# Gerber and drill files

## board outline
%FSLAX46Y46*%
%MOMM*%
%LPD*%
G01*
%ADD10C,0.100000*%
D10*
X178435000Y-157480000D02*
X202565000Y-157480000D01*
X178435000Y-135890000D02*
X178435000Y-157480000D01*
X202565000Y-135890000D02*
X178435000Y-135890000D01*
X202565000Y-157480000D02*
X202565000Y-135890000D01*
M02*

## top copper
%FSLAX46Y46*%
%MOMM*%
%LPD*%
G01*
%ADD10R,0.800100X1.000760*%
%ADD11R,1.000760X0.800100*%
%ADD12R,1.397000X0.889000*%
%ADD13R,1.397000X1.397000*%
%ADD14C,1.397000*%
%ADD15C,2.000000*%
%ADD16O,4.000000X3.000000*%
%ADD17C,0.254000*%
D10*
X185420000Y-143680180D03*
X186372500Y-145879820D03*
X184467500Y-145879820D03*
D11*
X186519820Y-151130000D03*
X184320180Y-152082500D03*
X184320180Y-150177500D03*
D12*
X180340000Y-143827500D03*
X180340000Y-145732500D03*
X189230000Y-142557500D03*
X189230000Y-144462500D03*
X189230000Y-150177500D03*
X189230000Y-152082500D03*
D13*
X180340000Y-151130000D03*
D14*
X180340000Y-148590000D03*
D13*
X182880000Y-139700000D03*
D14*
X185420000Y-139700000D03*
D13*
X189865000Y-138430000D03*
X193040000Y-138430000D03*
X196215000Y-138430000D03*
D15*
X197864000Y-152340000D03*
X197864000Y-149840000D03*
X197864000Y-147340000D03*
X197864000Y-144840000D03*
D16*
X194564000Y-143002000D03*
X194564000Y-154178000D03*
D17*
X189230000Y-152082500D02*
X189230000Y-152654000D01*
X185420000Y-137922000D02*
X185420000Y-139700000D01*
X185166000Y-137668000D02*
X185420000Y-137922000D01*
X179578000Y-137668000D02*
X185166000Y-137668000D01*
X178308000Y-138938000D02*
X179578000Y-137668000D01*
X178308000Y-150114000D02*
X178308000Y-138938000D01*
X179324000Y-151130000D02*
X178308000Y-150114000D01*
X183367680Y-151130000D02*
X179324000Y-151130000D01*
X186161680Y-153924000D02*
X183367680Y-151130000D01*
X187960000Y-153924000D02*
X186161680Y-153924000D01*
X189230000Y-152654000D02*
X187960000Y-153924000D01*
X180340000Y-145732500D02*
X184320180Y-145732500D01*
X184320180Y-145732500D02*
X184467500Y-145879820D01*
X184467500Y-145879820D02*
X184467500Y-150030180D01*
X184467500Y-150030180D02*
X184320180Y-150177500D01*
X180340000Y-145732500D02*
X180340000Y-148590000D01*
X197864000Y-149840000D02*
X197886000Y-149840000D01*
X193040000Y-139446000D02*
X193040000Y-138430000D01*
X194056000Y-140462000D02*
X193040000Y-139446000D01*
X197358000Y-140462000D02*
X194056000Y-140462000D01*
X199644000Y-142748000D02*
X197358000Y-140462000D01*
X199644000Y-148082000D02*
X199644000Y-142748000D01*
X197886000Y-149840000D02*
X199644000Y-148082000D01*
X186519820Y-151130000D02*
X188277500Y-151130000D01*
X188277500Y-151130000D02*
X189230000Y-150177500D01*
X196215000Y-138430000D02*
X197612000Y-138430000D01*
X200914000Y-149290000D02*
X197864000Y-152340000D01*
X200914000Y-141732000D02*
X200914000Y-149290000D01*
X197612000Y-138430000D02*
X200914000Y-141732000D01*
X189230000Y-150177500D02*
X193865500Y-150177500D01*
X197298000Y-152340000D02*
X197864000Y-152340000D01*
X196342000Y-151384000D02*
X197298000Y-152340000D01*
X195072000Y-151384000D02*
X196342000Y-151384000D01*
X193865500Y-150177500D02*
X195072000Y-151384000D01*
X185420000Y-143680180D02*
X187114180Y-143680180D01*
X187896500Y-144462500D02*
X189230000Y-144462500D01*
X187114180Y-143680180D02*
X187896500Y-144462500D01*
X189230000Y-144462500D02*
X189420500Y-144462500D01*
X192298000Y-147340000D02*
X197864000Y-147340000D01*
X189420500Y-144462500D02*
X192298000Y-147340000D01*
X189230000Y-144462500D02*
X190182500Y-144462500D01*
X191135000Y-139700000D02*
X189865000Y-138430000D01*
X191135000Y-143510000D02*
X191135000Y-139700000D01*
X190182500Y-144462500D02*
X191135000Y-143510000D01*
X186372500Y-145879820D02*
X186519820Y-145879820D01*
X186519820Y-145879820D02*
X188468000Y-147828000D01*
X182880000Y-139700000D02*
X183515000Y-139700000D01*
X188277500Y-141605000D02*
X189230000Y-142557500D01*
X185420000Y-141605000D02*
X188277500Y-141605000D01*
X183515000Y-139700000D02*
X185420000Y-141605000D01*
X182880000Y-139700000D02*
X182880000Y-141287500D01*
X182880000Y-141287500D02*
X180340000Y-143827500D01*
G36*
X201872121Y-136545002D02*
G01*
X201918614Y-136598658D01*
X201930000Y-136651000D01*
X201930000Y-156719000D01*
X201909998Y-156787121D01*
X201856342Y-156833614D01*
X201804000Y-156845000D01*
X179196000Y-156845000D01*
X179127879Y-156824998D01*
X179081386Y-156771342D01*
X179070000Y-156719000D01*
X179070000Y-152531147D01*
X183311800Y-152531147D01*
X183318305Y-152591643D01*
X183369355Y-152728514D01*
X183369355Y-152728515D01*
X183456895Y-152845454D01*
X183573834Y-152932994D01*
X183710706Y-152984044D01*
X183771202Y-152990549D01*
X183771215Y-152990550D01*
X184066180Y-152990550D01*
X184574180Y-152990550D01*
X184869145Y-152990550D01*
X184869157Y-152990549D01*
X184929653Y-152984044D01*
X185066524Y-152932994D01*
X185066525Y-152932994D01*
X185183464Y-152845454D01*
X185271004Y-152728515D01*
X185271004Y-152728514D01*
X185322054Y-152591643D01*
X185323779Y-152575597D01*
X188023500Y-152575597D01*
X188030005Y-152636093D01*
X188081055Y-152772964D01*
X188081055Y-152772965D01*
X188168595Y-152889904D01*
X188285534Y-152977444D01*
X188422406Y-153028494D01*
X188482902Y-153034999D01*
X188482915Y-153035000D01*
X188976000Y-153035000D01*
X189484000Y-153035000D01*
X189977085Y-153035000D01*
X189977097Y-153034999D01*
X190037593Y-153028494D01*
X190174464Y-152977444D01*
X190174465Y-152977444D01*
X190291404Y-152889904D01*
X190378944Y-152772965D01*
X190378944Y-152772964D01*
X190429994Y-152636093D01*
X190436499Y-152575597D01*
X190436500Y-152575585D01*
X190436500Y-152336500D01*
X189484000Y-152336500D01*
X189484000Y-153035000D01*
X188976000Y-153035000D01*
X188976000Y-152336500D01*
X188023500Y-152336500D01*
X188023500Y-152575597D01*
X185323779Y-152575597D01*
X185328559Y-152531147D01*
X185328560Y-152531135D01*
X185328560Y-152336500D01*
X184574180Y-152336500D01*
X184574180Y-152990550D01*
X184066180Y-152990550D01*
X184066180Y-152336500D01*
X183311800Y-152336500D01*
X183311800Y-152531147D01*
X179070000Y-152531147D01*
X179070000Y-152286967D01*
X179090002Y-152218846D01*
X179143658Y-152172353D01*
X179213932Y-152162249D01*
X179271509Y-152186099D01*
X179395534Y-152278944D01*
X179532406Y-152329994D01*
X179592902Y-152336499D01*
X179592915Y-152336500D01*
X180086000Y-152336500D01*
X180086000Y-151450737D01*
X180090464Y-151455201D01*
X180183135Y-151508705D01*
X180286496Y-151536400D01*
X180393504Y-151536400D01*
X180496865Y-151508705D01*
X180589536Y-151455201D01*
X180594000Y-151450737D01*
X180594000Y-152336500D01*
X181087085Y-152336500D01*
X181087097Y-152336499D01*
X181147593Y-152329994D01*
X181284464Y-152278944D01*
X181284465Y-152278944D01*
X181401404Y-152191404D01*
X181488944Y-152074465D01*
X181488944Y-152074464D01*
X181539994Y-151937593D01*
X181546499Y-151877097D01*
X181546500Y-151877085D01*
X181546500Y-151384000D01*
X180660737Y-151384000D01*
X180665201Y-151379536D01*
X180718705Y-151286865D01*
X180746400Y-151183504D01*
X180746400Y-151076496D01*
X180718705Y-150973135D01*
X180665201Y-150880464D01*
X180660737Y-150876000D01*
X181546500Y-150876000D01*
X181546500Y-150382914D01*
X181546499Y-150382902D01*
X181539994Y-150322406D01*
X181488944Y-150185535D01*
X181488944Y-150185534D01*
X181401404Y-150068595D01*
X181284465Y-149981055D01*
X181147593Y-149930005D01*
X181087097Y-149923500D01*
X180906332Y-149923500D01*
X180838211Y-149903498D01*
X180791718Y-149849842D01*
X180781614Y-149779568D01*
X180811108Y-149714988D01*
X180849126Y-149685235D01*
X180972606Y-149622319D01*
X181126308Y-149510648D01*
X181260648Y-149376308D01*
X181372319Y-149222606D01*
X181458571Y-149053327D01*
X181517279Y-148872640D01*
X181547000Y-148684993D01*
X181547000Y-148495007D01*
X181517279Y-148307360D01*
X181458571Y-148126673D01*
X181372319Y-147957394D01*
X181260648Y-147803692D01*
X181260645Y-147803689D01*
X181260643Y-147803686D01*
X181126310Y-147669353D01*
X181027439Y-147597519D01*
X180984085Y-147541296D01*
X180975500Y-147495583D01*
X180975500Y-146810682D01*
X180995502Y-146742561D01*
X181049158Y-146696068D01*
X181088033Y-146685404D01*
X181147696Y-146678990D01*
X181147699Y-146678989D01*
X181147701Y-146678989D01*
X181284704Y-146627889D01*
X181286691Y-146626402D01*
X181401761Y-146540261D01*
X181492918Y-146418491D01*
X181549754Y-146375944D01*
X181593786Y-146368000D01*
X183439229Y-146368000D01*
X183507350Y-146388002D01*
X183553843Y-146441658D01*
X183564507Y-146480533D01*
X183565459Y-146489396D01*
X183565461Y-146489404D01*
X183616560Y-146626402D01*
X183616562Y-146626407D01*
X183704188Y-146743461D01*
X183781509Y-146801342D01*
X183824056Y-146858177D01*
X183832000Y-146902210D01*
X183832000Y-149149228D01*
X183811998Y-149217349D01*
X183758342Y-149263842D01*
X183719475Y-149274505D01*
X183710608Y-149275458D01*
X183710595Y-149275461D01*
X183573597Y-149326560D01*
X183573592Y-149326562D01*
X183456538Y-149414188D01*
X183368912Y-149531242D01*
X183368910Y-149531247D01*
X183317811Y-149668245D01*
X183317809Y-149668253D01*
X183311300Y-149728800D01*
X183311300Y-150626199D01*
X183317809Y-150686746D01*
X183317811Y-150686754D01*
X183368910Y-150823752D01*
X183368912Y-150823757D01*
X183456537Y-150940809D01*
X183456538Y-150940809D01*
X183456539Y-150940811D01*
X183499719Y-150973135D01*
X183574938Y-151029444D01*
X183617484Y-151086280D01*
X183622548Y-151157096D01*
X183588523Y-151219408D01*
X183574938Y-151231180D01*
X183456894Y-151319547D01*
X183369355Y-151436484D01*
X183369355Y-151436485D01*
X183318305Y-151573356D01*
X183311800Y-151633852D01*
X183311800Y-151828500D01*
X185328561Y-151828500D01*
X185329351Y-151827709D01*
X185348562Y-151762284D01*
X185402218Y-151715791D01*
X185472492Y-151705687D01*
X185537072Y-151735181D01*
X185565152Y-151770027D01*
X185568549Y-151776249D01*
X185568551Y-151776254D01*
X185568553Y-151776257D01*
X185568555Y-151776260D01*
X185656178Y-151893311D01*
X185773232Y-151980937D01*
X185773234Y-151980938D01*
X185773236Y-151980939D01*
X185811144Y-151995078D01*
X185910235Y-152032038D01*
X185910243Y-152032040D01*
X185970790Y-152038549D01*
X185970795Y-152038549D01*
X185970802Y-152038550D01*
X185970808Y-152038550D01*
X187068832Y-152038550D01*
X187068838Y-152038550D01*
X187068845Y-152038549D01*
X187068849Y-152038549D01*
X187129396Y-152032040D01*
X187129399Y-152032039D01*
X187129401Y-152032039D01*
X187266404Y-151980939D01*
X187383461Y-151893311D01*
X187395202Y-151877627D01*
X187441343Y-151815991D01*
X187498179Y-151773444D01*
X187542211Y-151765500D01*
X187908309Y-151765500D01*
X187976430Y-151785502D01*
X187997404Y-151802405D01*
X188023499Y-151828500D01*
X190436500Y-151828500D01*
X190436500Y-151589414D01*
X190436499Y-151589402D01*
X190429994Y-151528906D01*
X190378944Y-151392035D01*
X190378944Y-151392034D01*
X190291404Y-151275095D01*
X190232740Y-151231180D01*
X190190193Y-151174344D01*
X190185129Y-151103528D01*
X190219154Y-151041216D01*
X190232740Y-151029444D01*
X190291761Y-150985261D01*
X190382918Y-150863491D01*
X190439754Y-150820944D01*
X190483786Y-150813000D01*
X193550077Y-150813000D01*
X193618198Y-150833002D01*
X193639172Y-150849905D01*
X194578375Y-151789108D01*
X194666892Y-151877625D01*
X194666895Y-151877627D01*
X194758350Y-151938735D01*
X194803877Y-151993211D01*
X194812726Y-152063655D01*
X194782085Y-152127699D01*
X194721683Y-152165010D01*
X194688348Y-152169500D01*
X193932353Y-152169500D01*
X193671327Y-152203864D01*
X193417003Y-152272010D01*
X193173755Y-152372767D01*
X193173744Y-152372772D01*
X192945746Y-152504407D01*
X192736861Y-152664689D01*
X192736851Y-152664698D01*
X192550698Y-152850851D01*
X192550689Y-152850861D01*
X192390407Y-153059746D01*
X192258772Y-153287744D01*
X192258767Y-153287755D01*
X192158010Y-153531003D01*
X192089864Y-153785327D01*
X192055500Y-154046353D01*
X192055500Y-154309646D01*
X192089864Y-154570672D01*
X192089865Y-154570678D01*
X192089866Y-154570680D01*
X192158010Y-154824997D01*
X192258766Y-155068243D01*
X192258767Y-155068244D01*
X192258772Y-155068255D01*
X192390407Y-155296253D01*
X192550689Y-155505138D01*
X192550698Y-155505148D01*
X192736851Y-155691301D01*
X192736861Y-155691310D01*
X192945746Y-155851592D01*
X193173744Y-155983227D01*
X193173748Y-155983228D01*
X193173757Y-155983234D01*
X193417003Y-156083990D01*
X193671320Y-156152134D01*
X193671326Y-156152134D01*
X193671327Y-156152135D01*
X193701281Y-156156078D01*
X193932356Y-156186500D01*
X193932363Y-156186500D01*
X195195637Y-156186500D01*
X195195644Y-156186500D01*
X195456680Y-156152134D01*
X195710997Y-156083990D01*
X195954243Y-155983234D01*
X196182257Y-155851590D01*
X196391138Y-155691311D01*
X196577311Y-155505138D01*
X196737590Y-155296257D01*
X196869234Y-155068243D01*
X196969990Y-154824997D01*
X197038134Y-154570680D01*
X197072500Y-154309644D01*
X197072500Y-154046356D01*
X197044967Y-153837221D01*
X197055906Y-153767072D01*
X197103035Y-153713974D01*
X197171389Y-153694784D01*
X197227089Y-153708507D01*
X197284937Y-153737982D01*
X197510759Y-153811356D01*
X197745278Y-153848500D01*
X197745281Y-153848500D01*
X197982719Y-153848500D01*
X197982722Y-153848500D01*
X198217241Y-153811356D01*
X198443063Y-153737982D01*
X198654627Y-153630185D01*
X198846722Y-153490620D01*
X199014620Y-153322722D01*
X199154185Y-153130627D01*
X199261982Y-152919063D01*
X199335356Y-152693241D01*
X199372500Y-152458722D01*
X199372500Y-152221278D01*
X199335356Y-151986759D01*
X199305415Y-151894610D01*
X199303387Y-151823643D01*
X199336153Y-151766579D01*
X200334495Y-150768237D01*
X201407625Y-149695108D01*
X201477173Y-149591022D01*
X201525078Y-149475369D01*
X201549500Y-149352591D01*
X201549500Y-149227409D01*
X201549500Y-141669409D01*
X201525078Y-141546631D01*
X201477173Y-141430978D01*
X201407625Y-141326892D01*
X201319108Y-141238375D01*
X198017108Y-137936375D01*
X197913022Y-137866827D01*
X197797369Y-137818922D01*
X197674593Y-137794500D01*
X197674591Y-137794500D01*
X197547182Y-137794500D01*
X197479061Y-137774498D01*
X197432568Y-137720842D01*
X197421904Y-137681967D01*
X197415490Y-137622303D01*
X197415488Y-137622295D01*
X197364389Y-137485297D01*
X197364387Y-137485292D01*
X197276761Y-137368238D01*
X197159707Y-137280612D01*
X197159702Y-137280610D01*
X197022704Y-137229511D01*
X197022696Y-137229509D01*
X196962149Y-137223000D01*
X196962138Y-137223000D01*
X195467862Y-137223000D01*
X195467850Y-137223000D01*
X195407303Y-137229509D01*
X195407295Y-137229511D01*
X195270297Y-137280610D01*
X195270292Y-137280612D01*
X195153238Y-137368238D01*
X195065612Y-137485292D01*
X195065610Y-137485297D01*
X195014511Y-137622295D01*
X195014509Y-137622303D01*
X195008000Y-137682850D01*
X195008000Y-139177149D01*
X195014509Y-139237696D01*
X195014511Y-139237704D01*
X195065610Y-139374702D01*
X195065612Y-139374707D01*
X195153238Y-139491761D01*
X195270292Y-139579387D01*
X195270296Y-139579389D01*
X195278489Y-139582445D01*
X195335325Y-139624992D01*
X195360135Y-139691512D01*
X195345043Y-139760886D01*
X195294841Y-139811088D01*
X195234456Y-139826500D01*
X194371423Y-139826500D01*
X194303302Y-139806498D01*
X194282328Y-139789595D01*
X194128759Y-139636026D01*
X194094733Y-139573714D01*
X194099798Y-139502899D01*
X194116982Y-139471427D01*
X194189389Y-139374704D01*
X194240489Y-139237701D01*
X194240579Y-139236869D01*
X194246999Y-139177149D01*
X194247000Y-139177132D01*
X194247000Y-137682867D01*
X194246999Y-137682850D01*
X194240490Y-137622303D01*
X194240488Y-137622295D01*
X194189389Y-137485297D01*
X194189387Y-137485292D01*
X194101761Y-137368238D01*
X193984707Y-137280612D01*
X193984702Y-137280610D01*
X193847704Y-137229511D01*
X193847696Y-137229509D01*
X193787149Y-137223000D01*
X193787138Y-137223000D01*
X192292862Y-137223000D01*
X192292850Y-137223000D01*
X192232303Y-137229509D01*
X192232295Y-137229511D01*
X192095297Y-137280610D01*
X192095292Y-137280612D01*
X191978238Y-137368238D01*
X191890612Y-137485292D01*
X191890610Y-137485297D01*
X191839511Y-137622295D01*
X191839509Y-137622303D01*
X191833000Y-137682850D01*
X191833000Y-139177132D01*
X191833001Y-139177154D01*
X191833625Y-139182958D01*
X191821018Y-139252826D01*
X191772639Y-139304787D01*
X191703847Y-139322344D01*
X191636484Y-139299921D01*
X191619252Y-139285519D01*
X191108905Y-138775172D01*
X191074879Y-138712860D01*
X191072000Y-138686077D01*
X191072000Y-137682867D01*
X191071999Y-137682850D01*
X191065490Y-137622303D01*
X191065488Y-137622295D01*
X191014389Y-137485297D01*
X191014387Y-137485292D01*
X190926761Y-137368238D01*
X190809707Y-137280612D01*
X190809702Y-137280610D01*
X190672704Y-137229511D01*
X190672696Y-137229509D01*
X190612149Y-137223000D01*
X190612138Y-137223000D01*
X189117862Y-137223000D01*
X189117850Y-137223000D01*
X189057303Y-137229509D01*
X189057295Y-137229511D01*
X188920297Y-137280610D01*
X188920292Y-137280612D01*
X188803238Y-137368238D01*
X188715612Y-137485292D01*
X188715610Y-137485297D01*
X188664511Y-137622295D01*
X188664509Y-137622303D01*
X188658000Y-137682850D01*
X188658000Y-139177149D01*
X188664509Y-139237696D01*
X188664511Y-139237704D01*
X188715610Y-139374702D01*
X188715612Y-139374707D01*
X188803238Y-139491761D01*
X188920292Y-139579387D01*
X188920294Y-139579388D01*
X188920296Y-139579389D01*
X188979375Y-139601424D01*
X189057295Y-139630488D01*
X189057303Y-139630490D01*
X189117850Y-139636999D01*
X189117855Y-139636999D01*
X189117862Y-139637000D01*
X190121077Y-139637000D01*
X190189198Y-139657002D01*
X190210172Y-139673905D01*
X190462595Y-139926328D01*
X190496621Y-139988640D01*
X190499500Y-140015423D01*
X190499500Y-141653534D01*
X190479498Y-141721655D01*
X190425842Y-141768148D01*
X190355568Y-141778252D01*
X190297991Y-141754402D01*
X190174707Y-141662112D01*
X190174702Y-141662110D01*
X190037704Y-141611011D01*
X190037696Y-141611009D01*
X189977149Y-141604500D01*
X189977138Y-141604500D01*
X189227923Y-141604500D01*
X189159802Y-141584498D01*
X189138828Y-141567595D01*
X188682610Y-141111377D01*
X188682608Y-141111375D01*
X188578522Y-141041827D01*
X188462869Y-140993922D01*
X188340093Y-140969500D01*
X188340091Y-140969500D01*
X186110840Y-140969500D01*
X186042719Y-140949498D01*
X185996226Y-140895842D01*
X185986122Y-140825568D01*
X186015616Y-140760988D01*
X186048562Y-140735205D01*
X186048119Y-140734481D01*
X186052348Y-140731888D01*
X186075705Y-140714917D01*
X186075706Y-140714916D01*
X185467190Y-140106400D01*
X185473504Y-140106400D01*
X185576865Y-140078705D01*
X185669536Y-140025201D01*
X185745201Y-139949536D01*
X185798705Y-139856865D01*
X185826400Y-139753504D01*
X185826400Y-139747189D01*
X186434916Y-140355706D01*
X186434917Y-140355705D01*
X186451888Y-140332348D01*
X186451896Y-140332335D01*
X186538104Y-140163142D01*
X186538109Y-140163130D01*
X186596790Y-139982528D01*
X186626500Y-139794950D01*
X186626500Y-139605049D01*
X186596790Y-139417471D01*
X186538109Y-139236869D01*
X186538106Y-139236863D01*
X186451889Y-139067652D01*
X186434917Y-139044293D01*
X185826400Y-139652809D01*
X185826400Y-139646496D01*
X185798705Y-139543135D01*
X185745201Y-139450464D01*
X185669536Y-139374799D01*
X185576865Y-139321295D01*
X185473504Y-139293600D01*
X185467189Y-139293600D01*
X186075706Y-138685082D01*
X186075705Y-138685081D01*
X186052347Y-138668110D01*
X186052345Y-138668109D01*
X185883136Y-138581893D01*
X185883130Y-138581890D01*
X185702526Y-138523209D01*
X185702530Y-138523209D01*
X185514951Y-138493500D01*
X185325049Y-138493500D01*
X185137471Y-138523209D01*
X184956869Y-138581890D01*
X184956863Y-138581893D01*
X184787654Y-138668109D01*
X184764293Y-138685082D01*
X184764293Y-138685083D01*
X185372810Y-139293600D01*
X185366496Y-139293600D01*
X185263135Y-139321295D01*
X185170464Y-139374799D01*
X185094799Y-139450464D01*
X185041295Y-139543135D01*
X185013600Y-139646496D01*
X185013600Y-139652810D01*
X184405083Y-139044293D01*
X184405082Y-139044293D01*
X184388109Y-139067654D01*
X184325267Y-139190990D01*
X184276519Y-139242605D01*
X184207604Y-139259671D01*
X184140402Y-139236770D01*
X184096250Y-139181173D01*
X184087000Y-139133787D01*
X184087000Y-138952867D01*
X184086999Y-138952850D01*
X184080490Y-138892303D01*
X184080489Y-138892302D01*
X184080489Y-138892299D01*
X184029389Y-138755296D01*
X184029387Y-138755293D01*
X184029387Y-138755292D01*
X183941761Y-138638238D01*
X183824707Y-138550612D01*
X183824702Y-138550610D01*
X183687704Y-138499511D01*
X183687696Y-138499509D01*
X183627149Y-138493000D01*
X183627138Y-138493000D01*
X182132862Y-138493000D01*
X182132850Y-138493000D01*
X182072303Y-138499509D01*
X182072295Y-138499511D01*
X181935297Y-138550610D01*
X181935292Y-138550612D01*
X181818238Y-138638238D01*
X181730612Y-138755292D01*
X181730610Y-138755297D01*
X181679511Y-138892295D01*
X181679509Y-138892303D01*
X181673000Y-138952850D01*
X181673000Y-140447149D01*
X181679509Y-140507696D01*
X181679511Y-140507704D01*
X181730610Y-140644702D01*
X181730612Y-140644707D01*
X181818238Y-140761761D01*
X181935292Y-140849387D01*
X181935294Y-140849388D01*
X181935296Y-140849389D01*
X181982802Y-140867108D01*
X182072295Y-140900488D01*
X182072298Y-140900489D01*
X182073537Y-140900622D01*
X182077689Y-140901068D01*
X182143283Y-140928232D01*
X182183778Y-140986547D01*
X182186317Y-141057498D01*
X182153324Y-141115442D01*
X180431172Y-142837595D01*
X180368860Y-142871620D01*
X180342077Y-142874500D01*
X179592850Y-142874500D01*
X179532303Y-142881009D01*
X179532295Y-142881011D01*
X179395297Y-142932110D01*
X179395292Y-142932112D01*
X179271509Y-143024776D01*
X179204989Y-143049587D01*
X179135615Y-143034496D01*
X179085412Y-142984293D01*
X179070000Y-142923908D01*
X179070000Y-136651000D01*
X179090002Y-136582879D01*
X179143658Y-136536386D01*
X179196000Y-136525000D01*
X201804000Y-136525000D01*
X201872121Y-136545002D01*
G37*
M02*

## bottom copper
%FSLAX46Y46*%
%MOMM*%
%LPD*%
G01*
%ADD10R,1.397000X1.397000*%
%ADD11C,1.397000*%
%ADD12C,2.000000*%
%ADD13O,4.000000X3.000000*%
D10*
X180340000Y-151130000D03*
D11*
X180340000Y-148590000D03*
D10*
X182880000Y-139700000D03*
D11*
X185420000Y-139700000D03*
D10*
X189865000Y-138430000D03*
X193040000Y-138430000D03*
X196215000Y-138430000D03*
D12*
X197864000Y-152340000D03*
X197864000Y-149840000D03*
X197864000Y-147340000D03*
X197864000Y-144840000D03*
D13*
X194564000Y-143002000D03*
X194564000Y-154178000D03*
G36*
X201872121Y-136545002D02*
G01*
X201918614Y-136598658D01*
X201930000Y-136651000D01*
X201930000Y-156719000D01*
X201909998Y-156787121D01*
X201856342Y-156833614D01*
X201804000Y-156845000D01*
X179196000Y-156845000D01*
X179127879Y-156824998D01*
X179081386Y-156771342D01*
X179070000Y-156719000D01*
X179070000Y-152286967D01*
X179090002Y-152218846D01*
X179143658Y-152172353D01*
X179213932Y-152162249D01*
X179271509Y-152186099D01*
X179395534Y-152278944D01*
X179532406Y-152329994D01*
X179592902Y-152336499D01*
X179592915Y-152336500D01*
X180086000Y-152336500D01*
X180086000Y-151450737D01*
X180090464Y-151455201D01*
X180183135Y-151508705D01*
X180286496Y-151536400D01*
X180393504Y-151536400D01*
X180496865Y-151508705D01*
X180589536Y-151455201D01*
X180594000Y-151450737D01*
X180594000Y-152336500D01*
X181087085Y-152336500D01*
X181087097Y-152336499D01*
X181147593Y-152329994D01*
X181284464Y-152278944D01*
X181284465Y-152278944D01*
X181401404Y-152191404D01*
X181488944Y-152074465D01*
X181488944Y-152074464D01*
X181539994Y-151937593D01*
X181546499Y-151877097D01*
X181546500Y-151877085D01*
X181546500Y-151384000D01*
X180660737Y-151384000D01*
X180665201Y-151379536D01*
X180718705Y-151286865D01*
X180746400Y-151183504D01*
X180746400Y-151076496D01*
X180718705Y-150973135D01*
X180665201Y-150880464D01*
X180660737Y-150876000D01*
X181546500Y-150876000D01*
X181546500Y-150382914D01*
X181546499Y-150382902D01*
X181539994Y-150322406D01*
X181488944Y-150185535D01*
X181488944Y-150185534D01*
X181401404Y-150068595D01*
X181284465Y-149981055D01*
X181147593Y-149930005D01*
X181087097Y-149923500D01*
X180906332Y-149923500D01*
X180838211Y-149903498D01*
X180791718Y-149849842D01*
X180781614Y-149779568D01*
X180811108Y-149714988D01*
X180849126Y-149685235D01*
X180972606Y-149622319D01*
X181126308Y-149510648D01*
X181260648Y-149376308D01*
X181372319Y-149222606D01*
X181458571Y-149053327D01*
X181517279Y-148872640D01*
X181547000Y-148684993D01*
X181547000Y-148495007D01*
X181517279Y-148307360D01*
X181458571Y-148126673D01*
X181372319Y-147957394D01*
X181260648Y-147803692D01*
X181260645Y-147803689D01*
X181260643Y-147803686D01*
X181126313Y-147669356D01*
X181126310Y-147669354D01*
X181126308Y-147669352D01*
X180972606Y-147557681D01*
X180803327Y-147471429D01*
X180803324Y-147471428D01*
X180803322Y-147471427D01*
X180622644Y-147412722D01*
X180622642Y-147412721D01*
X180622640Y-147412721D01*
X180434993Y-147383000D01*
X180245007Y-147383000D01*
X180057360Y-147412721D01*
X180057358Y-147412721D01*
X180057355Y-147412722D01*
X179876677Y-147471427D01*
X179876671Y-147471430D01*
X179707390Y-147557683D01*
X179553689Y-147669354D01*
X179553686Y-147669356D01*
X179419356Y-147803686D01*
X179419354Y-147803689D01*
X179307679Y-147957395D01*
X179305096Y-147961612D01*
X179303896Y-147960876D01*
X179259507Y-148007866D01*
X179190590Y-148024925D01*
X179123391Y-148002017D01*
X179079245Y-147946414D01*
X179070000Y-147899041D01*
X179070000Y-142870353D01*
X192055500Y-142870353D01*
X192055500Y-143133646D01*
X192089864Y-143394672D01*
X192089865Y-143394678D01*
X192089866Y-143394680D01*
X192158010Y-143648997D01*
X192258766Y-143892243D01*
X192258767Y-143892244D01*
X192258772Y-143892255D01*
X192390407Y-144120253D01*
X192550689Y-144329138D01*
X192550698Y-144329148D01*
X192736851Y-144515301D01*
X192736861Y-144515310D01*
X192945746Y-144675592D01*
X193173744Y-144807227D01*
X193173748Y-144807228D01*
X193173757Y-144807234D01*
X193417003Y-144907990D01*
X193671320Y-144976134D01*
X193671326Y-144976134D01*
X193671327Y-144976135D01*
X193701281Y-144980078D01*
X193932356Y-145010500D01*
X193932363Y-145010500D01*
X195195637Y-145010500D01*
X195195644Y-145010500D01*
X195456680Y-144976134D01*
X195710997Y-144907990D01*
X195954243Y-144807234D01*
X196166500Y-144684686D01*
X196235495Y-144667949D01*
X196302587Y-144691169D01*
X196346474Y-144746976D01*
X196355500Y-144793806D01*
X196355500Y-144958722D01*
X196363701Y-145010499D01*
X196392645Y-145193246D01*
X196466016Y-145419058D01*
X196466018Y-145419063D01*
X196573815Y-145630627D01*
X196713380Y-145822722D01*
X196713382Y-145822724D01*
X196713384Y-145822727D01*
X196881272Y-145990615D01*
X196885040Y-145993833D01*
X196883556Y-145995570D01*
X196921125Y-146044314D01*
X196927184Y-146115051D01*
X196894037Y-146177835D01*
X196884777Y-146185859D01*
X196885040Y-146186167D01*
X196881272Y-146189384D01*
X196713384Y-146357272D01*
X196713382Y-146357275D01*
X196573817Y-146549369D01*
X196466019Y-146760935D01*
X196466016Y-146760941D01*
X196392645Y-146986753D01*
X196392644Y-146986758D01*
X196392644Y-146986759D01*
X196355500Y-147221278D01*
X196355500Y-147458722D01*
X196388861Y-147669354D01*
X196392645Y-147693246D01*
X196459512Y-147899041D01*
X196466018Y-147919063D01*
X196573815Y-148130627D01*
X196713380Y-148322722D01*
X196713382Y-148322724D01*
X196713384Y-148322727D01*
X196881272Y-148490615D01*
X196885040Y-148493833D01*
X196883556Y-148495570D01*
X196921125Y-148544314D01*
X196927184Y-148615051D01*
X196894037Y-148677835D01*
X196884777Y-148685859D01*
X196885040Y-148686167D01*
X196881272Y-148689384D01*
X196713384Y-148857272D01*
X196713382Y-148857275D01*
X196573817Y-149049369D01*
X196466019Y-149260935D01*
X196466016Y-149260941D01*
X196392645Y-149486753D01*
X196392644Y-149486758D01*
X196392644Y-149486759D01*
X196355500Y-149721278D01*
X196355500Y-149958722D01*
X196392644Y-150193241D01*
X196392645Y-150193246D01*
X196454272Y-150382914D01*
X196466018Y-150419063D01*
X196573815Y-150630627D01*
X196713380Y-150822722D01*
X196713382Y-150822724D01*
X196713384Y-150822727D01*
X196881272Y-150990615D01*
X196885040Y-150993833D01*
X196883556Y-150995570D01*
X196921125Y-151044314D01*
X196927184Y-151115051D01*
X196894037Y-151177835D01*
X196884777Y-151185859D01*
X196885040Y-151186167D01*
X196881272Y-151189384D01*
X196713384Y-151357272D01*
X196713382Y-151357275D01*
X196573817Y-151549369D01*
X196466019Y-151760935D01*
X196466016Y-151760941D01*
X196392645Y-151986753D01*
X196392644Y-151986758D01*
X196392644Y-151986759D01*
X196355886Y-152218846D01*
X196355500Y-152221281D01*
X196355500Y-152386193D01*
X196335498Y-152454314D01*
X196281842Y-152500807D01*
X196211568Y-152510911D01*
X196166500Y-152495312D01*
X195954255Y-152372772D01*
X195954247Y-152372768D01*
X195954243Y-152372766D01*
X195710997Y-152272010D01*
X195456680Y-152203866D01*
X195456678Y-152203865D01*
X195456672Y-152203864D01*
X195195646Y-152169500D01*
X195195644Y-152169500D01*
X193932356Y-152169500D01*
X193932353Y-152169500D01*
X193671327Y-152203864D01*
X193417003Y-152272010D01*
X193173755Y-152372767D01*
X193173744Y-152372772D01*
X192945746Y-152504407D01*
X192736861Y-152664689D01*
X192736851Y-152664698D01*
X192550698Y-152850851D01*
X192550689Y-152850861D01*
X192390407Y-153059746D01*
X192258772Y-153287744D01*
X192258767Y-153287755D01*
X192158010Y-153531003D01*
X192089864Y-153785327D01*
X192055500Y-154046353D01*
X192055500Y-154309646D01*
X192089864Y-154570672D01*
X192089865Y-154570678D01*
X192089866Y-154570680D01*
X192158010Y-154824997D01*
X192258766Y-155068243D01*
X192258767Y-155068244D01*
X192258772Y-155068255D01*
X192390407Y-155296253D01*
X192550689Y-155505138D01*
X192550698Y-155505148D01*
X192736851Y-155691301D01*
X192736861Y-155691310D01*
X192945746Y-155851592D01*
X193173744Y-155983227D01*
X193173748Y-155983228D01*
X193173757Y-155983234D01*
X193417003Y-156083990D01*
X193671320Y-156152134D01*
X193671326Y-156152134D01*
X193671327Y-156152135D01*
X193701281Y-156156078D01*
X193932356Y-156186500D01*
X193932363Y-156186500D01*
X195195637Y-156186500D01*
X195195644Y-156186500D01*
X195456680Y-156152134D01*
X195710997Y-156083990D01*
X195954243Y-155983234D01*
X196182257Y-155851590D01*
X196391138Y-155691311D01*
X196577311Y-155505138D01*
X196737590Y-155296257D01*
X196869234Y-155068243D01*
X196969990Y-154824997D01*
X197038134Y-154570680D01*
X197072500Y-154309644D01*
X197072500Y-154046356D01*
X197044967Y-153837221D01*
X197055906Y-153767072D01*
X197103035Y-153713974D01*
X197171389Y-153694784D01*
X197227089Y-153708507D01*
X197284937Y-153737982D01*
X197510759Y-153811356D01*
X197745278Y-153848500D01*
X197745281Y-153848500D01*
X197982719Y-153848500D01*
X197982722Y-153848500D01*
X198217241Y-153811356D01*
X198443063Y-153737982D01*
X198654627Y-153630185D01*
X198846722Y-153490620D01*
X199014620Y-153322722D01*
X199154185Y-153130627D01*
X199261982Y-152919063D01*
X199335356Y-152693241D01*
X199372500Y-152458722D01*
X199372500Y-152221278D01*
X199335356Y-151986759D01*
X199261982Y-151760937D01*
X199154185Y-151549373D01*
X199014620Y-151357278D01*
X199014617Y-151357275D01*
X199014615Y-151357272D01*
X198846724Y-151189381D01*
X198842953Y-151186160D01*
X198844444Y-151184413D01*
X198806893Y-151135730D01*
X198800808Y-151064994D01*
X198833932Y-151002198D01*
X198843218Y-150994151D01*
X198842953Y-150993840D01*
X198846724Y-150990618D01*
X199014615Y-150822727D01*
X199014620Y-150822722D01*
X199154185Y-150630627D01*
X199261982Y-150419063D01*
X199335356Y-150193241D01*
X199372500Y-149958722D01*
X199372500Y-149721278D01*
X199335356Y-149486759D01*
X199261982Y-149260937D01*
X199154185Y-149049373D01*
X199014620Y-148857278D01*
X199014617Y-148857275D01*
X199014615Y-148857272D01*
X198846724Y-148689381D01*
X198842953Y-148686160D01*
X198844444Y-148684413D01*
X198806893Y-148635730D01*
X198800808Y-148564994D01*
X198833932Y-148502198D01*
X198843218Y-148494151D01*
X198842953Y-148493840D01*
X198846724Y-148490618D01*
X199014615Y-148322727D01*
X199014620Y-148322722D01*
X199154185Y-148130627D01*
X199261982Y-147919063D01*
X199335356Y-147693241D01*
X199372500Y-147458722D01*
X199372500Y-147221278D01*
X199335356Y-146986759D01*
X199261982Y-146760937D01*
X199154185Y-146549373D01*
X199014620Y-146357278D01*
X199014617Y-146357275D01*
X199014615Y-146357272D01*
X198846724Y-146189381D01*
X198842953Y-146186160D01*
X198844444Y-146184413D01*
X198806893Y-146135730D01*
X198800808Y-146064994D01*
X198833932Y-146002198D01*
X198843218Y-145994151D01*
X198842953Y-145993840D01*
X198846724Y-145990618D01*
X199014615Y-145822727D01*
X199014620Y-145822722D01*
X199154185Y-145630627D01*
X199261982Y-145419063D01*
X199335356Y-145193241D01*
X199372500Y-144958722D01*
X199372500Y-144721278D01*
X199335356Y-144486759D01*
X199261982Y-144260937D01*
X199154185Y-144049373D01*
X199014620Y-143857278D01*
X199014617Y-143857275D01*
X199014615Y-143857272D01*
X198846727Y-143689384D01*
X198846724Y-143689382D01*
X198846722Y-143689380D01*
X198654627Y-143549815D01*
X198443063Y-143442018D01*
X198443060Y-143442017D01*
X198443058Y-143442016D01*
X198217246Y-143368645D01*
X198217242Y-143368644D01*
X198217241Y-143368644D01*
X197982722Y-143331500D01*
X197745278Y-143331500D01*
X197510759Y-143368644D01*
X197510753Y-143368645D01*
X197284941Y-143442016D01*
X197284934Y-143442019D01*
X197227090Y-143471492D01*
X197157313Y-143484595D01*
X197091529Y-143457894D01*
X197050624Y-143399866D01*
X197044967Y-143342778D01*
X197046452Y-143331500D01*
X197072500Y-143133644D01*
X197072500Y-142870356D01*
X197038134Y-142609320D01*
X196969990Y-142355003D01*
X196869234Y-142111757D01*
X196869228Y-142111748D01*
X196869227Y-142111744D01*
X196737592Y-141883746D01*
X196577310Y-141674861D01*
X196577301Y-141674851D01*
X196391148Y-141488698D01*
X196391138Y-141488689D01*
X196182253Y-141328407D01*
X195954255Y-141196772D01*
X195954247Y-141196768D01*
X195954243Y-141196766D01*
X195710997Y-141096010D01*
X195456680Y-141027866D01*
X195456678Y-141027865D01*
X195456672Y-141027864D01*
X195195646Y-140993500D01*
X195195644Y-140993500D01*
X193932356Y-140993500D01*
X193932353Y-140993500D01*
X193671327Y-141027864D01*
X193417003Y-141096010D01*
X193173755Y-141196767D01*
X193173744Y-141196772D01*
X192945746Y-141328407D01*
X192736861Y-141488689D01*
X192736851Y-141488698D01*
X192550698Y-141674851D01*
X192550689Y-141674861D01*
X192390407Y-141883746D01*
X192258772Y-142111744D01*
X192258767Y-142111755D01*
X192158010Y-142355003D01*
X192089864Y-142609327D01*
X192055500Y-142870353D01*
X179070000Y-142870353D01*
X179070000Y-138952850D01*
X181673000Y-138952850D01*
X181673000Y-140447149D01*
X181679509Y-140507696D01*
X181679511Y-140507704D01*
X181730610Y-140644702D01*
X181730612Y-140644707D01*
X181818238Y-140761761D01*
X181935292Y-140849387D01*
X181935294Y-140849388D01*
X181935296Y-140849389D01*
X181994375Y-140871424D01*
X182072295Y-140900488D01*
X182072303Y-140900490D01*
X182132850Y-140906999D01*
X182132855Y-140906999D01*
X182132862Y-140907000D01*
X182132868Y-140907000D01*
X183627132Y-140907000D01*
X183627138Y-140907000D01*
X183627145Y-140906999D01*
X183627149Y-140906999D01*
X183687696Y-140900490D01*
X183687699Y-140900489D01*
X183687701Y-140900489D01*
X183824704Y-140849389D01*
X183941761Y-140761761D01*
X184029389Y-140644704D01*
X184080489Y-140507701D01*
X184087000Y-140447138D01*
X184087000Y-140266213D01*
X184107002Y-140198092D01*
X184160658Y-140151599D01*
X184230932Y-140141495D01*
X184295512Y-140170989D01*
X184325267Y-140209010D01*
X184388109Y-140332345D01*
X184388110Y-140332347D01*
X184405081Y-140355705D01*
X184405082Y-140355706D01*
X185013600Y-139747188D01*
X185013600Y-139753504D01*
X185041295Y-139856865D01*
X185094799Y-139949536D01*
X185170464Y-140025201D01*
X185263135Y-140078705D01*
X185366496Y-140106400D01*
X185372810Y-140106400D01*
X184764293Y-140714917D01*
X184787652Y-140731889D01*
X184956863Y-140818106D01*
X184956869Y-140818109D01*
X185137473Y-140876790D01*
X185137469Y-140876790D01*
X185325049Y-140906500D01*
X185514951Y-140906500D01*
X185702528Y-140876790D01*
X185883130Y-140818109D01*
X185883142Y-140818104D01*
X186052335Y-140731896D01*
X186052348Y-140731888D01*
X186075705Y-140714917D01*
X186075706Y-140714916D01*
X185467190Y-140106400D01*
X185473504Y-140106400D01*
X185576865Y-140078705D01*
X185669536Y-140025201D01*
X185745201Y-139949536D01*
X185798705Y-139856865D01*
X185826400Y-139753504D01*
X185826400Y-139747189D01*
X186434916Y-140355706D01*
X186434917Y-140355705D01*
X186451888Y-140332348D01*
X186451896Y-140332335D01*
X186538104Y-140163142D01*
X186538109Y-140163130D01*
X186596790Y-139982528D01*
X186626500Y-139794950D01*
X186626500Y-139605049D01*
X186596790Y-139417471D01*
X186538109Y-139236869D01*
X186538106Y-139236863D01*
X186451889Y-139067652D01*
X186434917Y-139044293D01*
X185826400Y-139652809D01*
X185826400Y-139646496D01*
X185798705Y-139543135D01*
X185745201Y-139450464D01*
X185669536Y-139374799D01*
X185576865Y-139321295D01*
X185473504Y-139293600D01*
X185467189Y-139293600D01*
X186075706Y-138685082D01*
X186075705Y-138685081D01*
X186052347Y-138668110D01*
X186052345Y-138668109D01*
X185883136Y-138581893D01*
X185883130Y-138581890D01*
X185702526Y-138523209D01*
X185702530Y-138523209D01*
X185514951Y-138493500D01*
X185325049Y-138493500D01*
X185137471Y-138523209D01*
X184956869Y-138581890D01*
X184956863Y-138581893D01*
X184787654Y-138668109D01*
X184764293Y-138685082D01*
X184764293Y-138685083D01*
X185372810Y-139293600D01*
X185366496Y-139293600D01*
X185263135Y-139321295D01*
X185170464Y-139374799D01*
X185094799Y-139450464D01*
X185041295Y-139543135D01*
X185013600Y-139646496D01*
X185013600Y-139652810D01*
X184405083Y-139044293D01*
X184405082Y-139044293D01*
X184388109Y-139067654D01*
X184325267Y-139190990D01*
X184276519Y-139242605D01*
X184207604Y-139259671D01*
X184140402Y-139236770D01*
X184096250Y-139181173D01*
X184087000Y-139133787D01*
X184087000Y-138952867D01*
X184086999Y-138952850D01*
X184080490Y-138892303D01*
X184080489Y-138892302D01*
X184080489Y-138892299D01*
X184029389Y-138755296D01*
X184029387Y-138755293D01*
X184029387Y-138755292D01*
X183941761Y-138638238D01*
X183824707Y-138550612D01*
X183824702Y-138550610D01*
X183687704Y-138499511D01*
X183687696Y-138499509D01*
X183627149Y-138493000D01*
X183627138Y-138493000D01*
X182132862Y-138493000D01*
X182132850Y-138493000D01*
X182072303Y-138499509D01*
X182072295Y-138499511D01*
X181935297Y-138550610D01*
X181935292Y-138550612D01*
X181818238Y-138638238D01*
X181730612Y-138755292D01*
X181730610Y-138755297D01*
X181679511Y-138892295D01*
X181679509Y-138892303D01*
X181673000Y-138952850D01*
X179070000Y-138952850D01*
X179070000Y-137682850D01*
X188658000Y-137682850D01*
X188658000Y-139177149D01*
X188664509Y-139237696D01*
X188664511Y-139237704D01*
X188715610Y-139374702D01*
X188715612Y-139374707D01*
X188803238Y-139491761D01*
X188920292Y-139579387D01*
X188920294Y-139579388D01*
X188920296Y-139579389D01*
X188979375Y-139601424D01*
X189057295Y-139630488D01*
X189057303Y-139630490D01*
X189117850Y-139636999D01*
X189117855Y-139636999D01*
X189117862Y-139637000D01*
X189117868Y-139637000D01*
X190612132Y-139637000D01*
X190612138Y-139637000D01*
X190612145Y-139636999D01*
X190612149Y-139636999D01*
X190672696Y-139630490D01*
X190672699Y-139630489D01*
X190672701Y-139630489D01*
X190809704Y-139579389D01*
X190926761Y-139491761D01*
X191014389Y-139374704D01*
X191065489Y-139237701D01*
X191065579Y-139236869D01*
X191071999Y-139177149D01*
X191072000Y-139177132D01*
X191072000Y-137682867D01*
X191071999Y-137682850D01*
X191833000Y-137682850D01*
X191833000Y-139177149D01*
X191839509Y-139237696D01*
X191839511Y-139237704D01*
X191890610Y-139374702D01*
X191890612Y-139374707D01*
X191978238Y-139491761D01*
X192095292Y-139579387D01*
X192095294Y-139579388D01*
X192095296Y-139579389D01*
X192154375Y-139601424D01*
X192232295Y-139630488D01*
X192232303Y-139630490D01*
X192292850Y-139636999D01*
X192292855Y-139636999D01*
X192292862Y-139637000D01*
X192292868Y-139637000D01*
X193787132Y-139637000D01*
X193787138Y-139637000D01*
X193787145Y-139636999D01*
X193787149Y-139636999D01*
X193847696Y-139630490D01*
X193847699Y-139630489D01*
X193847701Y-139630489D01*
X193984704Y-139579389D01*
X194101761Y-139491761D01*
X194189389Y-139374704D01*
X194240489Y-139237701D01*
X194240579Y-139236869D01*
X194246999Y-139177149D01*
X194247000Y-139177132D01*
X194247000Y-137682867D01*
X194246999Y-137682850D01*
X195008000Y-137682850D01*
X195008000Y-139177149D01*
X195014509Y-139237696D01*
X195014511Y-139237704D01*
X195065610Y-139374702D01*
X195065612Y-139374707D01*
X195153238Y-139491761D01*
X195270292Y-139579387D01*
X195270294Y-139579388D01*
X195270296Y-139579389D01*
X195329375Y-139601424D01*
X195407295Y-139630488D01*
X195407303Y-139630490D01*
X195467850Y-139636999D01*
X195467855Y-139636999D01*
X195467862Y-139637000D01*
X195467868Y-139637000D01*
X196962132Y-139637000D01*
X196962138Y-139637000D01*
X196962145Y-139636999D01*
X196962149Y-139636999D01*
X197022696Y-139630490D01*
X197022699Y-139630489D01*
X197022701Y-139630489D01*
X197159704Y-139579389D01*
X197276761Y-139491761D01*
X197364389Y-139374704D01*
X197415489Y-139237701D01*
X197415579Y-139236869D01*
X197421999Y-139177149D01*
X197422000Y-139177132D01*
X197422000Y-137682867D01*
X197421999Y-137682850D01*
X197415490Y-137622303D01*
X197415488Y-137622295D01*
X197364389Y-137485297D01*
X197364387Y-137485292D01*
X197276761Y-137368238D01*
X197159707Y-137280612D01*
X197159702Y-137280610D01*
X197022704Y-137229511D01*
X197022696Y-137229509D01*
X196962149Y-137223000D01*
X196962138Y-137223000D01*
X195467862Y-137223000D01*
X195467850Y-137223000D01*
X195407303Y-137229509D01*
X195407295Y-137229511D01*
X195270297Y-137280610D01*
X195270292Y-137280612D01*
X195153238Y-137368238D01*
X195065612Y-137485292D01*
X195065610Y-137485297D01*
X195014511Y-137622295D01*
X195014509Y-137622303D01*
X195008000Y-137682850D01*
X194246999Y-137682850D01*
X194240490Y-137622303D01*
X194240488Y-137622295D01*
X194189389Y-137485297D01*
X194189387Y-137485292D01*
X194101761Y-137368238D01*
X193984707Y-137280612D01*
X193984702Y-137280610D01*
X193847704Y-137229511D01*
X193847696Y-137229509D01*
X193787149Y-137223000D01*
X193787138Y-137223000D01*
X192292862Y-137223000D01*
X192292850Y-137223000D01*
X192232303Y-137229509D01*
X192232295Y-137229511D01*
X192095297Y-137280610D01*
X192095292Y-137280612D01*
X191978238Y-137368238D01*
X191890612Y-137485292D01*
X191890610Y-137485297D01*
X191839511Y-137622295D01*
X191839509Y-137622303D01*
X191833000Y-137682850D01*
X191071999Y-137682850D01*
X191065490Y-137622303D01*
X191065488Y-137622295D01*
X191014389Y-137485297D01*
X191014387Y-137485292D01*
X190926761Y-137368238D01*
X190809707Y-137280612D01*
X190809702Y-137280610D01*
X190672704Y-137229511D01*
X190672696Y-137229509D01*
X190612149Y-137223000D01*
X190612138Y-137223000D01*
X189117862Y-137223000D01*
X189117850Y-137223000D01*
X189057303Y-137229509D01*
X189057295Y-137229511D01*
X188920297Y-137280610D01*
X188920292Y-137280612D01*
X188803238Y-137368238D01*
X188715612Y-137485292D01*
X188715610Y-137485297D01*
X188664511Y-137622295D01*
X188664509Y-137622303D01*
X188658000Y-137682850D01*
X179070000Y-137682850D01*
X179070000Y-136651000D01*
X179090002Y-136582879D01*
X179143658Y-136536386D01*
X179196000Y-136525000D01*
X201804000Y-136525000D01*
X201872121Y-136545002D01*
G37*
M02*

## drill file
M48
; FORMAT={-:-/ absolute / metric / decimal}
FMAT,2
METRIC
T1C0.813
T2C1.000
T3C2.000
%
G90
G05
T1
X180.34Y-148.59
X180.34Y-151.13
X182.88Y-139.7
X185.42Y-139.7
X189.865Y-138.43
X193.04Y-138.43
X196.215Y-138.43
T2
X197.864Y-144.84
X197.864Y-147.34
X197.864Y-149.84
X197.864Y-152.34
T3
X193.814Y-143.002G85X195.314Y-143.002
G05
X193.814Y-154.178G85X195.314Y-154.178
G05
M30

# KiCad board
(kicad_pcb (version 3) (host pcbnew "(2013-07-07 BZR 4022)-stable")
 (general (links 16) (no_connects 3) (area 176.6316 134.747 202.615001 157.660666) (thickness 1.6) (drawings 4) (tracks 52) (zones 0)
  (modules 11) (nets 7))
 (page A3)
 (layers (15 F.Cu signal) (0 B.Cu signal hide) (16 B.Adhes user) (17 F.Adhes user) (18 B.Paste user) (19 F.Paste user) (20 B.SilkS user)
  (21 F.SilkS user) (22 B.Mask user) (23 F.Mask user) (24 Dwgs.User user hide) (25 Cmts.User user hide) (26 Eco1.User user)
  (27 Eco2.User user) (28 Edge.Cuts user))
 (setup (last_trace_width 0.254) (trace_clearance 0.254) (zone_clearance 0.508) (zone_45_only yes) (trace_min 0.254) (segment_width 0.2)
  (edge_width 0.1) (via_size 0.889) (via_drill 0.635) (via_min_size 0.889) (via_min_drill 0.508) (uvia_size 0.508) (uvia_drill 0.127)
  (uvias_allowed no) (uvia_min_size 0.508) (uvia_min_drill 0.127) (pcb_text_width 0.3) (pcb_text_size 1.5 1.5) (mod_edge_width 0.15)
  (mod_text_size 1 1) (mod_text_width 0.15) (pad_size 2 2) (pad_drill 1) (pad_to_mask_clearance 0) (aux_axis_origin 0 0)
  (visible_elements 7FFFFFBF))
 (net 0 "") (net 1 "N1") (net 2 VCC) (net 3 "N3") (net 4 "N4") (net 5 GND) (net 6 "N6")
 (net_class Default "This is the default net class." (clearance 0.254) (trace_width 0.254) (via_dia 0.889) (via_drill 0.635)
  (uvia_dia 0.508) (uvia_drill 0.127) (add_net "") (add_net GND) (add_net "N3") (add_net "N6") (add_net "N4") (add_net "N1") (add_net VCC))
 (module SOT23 (layer F.Cu) (at 185.42 144.78)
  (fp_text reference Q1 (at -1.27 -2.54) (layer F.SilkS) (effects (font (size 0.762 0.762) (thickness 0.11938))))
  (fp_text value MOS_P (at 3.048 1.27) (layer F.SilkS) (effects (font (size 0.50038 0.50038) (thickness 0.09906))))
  (pad D smd rect (at 0 -1.09982) (size 0.8001 1.00076) (layers F.Cu F.Paste F.Mask) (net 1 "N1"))
  (pad S smd rect (at 0.9525 1.09982) (size 0.8001 1.00076) (layers F.Cu F.Paste F.Mask) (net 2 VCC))
  (pad G smd rect (at -0.9525 1.09982) (size 0.8001 1.00076) (layers F.Cu F.Paste F.Mask) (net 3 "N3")))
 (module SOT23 (layer F.Cu) (at 185.42 151.13 270)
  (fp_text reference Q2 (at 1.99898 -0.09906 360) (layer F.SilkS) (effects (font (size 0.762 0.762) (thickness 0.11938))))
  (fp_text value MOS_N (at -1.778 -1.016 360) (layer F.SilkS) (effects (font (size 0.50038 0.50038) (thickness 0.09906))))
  (pad D smd rect (at 0 -1.09982 270) (size 0.8001 1.00076) (layers F.Cu F.Paste F.Mask) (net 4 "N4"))
  (pad S smd rect (at 0.9525 1.09982 270) (size 0.8001 1.00076) (layers F.Cu F.Paste F.Mask) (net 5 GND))
  (pad G smd rect (at -0.9525 1.09982 270) (size 0.8001 1.00076) (layers F.Cu F.Paste F.Mask) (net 3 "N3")))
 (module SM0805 (layer F.Cu) (at 180.34 144.78 270)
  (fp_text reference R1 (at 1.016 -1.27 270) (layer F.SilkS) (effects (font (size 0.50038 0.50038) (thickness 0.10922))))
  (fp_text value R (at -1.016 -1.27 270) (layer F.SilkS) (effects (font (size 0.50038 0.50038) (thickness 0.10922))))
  (pad 1 smd rect (at -0.9525 0 270) (size 0.889 1.397) (layers F.Cu F.Paste F.Mask) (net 2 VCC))
  (pad 2 smd rect (at 0.9525 0 270) (size 0.889 1.397) (layers F.Cu F.Paste F.Mask) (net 3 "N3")))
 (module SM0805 (layer F.Cu) (at 189.23 143.51 270)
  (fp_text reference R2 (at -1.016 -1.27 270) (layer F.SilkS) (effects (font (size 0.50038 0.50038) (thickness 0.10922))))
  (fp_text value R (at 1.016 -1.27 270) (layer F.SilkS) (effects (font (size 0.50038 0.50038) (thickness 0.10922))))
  (pad 1 smd rect (at -0.9525 0 270) (size 0.889 1.397) (layers F.Cu F.Paste F.Mask) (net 2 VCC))
  (pad 2 smd rect (at 0.9525 0 270) (size 0.889 1.397) (layers F.Cu F.Paste F.Mask) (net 1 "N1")))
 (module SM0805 (layer F.Cu) (at 189.23 151.13 270)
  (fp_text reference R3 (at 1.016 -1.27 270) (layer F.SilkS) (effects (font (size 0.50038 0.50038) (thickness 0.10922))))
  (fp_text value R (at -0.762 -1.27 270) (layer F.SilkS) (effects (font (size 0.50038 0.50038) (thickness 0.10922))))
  (pad 1 smd rect (at -0.9525 0 270) (size 0.889 1.397) (layers F.Cu F.Paste F.Mask) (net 4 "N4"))
  (pad 2 smd rect (at 0.9525 0 270) (size 0.889 1.397) (layers F.Cu F.Paste F.Mask) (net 5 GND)))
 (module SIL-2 (layer F.Cu) (at 180.34 149.86 90)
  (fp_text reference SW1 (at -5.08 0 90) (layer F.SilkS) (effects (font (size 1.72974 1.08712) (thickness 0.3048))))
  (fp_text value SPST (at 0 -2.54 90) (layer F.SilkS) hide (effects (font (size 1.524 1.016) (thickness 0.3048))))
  (pad 1 thru_hole rect (at -1.27 0 90) (size 1.397 1.397) (drill 0.8128) (layers *.Cu *.Mask F.SilkS) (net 5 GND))
  (pad 2 thru_hole circle (at 1.27 0 90) (size 1.397 1.397) (drill 0.8128) (layers *.Cu *.Mask F.SilkS) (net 3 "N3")))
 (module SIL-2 (layer F.Cu) (at 184.15 139.7)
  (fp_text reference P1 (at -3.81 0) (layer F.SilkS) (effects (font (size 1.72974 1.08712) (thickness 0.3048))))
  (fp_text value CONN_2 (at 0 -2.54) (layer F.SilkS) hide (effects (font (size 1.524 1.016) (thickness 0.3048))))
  (pad 1 thru_hole rect (at -1.27 0) (size 1.397 1.397) (drill 0.8128) (layers *.Cu *.Mask F.SilkS) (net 2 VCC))
  (pad 2 thru_hole circle (at 1.27 0) (size 1.397 1.397) (drill 0.8128) (layers *.Cu *.Mask F.SilkS) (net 5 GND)))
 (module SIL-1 (layer F.Cu) (at 189.865 138.43)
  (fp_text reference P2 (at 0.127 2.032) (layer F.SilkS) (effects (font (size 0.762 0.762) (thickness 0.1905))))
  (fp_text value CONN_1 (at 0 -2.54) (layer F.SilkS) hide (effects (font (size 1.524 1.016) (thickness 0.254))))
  (pad 1 thru_hole rect (at 0 0) (size 1.397 1.397) (drill 0.8128) (layers *.Cu *.Mask F.SilkS) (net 1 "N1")))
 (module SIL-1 (layer F.Cu) (at 193.04 138.43)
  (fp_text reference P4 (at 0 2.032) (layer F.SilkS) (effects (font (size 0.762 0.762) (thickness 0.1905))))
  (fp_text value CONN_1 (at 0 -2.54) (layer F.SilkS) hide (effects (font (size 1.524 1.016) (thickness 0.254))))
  (pad 1 thru_hole rect (at 0 0) (size 1.397 1.397) (drill 0.8128) (layers *.Cu *.Mask F.SilkS) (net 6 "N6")))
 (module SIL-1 (layer F.Cu) (at 196.215 138.43)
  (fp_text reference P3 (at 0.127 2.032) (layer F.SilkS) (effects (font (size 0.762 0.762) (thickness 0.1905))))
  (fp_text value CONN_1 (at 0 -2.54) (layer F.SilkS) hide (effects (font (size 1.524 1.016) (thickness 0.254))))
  (pad 1 thru_hole rect (at 0 0) (size 1.397 1.397) (drill 0.8128) (layers *.Cu *.Mask F.SilkS) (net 4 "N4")))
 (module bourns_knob (layer F.Cu) (at 194.564 148.59 90)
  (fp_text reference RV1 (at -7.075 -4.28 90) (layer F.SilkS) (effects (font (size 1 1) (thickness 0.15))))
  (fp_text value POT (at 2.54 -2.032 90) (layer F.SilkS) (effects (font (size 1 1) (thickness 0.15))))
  (pad 3 thru_hole circle (at -3.75 3.3 90) (size 2 2) (drill 1) (layers *.Cu *.Mask F.SilkS) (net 4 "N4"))
  (pad 2 thru_hole circle (at -1.25 3.3 90) (size 2 2) (drill 1) (layers *.Cu *.Mask F.SilkS) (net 6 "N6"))
  (pad 1 thru_hole circle (at 1.25 3.3 90) (size 2 2) (drill 1) (layers *.Cu *.Mask F.SilkS) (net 1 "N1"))
  (pad 4 thru_hole circle (at 3.75 3.3 90) (size 2 2) (drill 1) (layers *.Cu *.Mask F.SilkS))
  (pad "" thru_hole oval (at 5.588 0 90) (size 3 4) (drill oval 2 3.5) (layers *.Cu *.Mask F.SilkS))
  (pad "" thru_hole oval (at -5.588 0 90) (size 3 4) (drill oval 2 3.5) (layers *.Cu *.Mask F.SilkS)))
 (gr_line (start 178.435 157.48) (end 202.565 157.48) (angle 90) (layer Edge.Cuts) (width 0.1))
 (gr_line (start 178.435 135.89) (end 178.435 157.48) (angle 90) (layer Edge.Cuts) (width 0.1))
 (gr_line (start 202.565 135.89) (end 178.435 135.89) (angle 90) (layer Edge.Cuts) (width 0.1))
 (gr_line (start 202.565 157.48) (end 202.565 135.89) (angle 90) (layer Edge.Cuts) (width 0.1))
 (segment (start 189.23 152.0825) (end 189.23 152.654) (width 0.254) (layer F.Cu) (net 5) (status 400000))
 (segment (start 185.42 137.922) (end 185.42 139.7) (width 0.254) (layer F.Cu) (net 5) (status 800000))
 (segment (start 185.166 137.668) (end 185.42 137.922) (width 0.254) (layer F.Cu) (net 5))
 (segment (start 179.578 137.668) (end 185.166 137.668) (width 0.254) (layer F.Cu) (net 5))
 (segment (start 178.308 138.938) (end 179.578 137.668) (width 0.254) (layer F.Cu) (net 5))
 (segment (start 178.308 150.114) (end 178.308 138.938) (width 0.254) (layer F.Cu) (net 5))
 (segment (start 179.324 151.13) (end 178.308 150.114) (width 0.254) (layer F.Cu) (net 5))
 (segment (start 183.36768 151.13) (end 179.324 151.13) (width 0.254) (layer F.Cu) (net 5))
 (segment (start 186.16168 153.924) (end 183.36768 151.13) (width 0.254) (layer F.Cu) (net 5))
 (segment (start 187.96 153.924) (end 186.16168 153.924) (width 0.254) (layer F.Cu) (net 5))
 (segment (start 189.23 152.654) (end 187.96 153.924) (width 0.254) (layer F.Cu) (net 5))
 (segment (start 180.34 145.7325) (end 184.32018 145.7325) (width 0.254) (layer F.Cu) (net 3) (status C00000))
 (segment (start 184.32018 145.7325) (end 184.4675 145.87982) (width 0.254) (layer F.Cu) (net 3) (status C00000))
 (segment (start 184.4675 145.87982) (end 184.4675 150.03018) (width 0.254) (layer F.Cu) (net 3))
 (segment (start 184.4675 150.03018) (end 184.32018 150.1775) (width 0.254) (layer F.Cu) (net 3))
 (segment (start 180.34 145.7325) (end 180.34 148.59) (width 0.254) (layer F.Cu) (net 3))
 (segment (start 197.864 149.84) (end 197.886 149.84) (width 0.254) (layer F.Cu) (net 6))
 (segment (start 193.04 139.446) (end 193.04 138.43) (width 0.254) (layer F.Cu) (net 6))
 (segment (start 194.056 140.462) (end 193.04 139.446) (width 0.254) (layer F.Cu) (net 6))
 (segment (start 197.358 140.462) (end 194.056 140.462) (width 0.254) (layer F.Cu) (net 6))
 (segment (start 199.644 142.748) (end 197.358 140.462) (width 0.254) (layer F.Cu) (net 6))
 (segment (start 199.644 148.082) (end 199.644 142.748) (width 0.254) (layer F.Cu) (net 6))
 (segment (start 197.886 149.84) (end 199.644 148.082) (width 0.254) (layer F.Cu) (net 6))
 (segment (start 186.51982 151.13) (end 188.2775 151.13) (width 0.254) (layer F.Cu) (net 4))
 (segment (start 188.2775 151.13) (end 189.23 150.1775) (width 0.254) (layer F.Cu) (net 4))
 (segment (start 196.215 138.43) (end 197.612 138.43) (width 0.254) (layer F.Cu) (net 4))
 (segment (start 200.914 149.29) (end 197.864 152.34) (width 0.254) (layer F.Cu) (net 4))
 (segment (start 200.914 141.732) (end 200.914 149.29) (width 0.254) (layer F.Cu) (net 4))
 (segment (start 197.612 138.43) (end 200.914 141.732) (width 0.254) (layer F.Cu) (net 4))
 (segment (start 189.23 150.1775) (end 193.8655 150.1775) (width 0.254) (layer F.Cu) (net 4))
 (segment (start 197.298 152.34) (end 197.864 152.34) (width 0.254) (layer F.Cu) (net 4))
 (segment (start 196.342 151.384) (end 197.298 152.34) (width 0.254) (layer F.Cu) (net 4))
 (segment (start 195.072 151.384) (end 196.342 151.384) (width 0.254) (layer F.Cu) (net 4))
 (segment (start 193.8655 150.1775) (end 195.072 151.384) (width 0.254) (layer F.Cu) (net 4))
 (segment (start 185.42 143.68018) (end 187.11418 143.68018) (width 0.254) (layer F.Cu) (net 1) (status 400000))
 (segment (start 187.8965 144.4625) (end 189.23 144.4625) (width 0.254) (layer F.Cu) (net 1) (status 800000))
 (segment (start 187.11418 143.68018) (end 187.8965 144.4625) (width 0.254) (layer F.Cu) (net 1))
 (segment (start 189.23 144.4625) (end 189.4205 144.4625) (width 0.254) (layer F.Cu) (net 1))
 (segment (start 192.298 147.34) (end 197.864 147.34) (width 0.254) (layer F.Cu) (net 1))
 (segment (start 189.4205 144.4625) (end 192.298 147.34) (width 0.254) (layer F.Cu) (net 1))
 (segment (start 189.23 144.4625) (end 190.1825 144.4625) (width 0.254) (layer F.Cu) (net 1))
 (segment (start 191.135 139.7) (end 189.865 138.43) (width 0.254) (layer F.Cu) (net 1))
 (segment (start 191.135 143.51) (end 191.135 139.7) (width 0.254) (layer F.Cu) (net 1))
 (segment (start 190.1825 144.4625) (end 191.135 143.51) (width 0.254) (layer F.Cu) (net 1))
 (segment (start 186.3725 145.87982) (end 186.51982 145.87982) (width 0.254) (layer F.Cu) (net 2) (status C00000))
 (segment (start 186.51982 145.87982) (end 188.468 147.828) (width 0.254) (layer F.Cu) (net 2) (status 400000))
 (segment (start 182.88 139.7) (end 183.515 139.7) (width 0.254) (layer F.Cu) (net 2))
 (segment (start 188.2775 141.605) (end 189.23 142.5575) (width 0.254) (layer F.Cu) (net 2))
 (segment (start 185.42 141.605) (end 188.2775 141.605) (width 0.254) (layer F.Cu) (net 2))
 (segment (start 183.515 139.7) (end 185.42 141.605) (width 0.254) (layer F.Cu) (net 2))
 (segment (start 182.88 139.7) (end 182.88 141.2875) (width 0.254) (layer F.Cu) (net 2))
 (segment (start 182.88 141.2875) (end 180.34 143.8275) (width 0.254) (layer F.Cu) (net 2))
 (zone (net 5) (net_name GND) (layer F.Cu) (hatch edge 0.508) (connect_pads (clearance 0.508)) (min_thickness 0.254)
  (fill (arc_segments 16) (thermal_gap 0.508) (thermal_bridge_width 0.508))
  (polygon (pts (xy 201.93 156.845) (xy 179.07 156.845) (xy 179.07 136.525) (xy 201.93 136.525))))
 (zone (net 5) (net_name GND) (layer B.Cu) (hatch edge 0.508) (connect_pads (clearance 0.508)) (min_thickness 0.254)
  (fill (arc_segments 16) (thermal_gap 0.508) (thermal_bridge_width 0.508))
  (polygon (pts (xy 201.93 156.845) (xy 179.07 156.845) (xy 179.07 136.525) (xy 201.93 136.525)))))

